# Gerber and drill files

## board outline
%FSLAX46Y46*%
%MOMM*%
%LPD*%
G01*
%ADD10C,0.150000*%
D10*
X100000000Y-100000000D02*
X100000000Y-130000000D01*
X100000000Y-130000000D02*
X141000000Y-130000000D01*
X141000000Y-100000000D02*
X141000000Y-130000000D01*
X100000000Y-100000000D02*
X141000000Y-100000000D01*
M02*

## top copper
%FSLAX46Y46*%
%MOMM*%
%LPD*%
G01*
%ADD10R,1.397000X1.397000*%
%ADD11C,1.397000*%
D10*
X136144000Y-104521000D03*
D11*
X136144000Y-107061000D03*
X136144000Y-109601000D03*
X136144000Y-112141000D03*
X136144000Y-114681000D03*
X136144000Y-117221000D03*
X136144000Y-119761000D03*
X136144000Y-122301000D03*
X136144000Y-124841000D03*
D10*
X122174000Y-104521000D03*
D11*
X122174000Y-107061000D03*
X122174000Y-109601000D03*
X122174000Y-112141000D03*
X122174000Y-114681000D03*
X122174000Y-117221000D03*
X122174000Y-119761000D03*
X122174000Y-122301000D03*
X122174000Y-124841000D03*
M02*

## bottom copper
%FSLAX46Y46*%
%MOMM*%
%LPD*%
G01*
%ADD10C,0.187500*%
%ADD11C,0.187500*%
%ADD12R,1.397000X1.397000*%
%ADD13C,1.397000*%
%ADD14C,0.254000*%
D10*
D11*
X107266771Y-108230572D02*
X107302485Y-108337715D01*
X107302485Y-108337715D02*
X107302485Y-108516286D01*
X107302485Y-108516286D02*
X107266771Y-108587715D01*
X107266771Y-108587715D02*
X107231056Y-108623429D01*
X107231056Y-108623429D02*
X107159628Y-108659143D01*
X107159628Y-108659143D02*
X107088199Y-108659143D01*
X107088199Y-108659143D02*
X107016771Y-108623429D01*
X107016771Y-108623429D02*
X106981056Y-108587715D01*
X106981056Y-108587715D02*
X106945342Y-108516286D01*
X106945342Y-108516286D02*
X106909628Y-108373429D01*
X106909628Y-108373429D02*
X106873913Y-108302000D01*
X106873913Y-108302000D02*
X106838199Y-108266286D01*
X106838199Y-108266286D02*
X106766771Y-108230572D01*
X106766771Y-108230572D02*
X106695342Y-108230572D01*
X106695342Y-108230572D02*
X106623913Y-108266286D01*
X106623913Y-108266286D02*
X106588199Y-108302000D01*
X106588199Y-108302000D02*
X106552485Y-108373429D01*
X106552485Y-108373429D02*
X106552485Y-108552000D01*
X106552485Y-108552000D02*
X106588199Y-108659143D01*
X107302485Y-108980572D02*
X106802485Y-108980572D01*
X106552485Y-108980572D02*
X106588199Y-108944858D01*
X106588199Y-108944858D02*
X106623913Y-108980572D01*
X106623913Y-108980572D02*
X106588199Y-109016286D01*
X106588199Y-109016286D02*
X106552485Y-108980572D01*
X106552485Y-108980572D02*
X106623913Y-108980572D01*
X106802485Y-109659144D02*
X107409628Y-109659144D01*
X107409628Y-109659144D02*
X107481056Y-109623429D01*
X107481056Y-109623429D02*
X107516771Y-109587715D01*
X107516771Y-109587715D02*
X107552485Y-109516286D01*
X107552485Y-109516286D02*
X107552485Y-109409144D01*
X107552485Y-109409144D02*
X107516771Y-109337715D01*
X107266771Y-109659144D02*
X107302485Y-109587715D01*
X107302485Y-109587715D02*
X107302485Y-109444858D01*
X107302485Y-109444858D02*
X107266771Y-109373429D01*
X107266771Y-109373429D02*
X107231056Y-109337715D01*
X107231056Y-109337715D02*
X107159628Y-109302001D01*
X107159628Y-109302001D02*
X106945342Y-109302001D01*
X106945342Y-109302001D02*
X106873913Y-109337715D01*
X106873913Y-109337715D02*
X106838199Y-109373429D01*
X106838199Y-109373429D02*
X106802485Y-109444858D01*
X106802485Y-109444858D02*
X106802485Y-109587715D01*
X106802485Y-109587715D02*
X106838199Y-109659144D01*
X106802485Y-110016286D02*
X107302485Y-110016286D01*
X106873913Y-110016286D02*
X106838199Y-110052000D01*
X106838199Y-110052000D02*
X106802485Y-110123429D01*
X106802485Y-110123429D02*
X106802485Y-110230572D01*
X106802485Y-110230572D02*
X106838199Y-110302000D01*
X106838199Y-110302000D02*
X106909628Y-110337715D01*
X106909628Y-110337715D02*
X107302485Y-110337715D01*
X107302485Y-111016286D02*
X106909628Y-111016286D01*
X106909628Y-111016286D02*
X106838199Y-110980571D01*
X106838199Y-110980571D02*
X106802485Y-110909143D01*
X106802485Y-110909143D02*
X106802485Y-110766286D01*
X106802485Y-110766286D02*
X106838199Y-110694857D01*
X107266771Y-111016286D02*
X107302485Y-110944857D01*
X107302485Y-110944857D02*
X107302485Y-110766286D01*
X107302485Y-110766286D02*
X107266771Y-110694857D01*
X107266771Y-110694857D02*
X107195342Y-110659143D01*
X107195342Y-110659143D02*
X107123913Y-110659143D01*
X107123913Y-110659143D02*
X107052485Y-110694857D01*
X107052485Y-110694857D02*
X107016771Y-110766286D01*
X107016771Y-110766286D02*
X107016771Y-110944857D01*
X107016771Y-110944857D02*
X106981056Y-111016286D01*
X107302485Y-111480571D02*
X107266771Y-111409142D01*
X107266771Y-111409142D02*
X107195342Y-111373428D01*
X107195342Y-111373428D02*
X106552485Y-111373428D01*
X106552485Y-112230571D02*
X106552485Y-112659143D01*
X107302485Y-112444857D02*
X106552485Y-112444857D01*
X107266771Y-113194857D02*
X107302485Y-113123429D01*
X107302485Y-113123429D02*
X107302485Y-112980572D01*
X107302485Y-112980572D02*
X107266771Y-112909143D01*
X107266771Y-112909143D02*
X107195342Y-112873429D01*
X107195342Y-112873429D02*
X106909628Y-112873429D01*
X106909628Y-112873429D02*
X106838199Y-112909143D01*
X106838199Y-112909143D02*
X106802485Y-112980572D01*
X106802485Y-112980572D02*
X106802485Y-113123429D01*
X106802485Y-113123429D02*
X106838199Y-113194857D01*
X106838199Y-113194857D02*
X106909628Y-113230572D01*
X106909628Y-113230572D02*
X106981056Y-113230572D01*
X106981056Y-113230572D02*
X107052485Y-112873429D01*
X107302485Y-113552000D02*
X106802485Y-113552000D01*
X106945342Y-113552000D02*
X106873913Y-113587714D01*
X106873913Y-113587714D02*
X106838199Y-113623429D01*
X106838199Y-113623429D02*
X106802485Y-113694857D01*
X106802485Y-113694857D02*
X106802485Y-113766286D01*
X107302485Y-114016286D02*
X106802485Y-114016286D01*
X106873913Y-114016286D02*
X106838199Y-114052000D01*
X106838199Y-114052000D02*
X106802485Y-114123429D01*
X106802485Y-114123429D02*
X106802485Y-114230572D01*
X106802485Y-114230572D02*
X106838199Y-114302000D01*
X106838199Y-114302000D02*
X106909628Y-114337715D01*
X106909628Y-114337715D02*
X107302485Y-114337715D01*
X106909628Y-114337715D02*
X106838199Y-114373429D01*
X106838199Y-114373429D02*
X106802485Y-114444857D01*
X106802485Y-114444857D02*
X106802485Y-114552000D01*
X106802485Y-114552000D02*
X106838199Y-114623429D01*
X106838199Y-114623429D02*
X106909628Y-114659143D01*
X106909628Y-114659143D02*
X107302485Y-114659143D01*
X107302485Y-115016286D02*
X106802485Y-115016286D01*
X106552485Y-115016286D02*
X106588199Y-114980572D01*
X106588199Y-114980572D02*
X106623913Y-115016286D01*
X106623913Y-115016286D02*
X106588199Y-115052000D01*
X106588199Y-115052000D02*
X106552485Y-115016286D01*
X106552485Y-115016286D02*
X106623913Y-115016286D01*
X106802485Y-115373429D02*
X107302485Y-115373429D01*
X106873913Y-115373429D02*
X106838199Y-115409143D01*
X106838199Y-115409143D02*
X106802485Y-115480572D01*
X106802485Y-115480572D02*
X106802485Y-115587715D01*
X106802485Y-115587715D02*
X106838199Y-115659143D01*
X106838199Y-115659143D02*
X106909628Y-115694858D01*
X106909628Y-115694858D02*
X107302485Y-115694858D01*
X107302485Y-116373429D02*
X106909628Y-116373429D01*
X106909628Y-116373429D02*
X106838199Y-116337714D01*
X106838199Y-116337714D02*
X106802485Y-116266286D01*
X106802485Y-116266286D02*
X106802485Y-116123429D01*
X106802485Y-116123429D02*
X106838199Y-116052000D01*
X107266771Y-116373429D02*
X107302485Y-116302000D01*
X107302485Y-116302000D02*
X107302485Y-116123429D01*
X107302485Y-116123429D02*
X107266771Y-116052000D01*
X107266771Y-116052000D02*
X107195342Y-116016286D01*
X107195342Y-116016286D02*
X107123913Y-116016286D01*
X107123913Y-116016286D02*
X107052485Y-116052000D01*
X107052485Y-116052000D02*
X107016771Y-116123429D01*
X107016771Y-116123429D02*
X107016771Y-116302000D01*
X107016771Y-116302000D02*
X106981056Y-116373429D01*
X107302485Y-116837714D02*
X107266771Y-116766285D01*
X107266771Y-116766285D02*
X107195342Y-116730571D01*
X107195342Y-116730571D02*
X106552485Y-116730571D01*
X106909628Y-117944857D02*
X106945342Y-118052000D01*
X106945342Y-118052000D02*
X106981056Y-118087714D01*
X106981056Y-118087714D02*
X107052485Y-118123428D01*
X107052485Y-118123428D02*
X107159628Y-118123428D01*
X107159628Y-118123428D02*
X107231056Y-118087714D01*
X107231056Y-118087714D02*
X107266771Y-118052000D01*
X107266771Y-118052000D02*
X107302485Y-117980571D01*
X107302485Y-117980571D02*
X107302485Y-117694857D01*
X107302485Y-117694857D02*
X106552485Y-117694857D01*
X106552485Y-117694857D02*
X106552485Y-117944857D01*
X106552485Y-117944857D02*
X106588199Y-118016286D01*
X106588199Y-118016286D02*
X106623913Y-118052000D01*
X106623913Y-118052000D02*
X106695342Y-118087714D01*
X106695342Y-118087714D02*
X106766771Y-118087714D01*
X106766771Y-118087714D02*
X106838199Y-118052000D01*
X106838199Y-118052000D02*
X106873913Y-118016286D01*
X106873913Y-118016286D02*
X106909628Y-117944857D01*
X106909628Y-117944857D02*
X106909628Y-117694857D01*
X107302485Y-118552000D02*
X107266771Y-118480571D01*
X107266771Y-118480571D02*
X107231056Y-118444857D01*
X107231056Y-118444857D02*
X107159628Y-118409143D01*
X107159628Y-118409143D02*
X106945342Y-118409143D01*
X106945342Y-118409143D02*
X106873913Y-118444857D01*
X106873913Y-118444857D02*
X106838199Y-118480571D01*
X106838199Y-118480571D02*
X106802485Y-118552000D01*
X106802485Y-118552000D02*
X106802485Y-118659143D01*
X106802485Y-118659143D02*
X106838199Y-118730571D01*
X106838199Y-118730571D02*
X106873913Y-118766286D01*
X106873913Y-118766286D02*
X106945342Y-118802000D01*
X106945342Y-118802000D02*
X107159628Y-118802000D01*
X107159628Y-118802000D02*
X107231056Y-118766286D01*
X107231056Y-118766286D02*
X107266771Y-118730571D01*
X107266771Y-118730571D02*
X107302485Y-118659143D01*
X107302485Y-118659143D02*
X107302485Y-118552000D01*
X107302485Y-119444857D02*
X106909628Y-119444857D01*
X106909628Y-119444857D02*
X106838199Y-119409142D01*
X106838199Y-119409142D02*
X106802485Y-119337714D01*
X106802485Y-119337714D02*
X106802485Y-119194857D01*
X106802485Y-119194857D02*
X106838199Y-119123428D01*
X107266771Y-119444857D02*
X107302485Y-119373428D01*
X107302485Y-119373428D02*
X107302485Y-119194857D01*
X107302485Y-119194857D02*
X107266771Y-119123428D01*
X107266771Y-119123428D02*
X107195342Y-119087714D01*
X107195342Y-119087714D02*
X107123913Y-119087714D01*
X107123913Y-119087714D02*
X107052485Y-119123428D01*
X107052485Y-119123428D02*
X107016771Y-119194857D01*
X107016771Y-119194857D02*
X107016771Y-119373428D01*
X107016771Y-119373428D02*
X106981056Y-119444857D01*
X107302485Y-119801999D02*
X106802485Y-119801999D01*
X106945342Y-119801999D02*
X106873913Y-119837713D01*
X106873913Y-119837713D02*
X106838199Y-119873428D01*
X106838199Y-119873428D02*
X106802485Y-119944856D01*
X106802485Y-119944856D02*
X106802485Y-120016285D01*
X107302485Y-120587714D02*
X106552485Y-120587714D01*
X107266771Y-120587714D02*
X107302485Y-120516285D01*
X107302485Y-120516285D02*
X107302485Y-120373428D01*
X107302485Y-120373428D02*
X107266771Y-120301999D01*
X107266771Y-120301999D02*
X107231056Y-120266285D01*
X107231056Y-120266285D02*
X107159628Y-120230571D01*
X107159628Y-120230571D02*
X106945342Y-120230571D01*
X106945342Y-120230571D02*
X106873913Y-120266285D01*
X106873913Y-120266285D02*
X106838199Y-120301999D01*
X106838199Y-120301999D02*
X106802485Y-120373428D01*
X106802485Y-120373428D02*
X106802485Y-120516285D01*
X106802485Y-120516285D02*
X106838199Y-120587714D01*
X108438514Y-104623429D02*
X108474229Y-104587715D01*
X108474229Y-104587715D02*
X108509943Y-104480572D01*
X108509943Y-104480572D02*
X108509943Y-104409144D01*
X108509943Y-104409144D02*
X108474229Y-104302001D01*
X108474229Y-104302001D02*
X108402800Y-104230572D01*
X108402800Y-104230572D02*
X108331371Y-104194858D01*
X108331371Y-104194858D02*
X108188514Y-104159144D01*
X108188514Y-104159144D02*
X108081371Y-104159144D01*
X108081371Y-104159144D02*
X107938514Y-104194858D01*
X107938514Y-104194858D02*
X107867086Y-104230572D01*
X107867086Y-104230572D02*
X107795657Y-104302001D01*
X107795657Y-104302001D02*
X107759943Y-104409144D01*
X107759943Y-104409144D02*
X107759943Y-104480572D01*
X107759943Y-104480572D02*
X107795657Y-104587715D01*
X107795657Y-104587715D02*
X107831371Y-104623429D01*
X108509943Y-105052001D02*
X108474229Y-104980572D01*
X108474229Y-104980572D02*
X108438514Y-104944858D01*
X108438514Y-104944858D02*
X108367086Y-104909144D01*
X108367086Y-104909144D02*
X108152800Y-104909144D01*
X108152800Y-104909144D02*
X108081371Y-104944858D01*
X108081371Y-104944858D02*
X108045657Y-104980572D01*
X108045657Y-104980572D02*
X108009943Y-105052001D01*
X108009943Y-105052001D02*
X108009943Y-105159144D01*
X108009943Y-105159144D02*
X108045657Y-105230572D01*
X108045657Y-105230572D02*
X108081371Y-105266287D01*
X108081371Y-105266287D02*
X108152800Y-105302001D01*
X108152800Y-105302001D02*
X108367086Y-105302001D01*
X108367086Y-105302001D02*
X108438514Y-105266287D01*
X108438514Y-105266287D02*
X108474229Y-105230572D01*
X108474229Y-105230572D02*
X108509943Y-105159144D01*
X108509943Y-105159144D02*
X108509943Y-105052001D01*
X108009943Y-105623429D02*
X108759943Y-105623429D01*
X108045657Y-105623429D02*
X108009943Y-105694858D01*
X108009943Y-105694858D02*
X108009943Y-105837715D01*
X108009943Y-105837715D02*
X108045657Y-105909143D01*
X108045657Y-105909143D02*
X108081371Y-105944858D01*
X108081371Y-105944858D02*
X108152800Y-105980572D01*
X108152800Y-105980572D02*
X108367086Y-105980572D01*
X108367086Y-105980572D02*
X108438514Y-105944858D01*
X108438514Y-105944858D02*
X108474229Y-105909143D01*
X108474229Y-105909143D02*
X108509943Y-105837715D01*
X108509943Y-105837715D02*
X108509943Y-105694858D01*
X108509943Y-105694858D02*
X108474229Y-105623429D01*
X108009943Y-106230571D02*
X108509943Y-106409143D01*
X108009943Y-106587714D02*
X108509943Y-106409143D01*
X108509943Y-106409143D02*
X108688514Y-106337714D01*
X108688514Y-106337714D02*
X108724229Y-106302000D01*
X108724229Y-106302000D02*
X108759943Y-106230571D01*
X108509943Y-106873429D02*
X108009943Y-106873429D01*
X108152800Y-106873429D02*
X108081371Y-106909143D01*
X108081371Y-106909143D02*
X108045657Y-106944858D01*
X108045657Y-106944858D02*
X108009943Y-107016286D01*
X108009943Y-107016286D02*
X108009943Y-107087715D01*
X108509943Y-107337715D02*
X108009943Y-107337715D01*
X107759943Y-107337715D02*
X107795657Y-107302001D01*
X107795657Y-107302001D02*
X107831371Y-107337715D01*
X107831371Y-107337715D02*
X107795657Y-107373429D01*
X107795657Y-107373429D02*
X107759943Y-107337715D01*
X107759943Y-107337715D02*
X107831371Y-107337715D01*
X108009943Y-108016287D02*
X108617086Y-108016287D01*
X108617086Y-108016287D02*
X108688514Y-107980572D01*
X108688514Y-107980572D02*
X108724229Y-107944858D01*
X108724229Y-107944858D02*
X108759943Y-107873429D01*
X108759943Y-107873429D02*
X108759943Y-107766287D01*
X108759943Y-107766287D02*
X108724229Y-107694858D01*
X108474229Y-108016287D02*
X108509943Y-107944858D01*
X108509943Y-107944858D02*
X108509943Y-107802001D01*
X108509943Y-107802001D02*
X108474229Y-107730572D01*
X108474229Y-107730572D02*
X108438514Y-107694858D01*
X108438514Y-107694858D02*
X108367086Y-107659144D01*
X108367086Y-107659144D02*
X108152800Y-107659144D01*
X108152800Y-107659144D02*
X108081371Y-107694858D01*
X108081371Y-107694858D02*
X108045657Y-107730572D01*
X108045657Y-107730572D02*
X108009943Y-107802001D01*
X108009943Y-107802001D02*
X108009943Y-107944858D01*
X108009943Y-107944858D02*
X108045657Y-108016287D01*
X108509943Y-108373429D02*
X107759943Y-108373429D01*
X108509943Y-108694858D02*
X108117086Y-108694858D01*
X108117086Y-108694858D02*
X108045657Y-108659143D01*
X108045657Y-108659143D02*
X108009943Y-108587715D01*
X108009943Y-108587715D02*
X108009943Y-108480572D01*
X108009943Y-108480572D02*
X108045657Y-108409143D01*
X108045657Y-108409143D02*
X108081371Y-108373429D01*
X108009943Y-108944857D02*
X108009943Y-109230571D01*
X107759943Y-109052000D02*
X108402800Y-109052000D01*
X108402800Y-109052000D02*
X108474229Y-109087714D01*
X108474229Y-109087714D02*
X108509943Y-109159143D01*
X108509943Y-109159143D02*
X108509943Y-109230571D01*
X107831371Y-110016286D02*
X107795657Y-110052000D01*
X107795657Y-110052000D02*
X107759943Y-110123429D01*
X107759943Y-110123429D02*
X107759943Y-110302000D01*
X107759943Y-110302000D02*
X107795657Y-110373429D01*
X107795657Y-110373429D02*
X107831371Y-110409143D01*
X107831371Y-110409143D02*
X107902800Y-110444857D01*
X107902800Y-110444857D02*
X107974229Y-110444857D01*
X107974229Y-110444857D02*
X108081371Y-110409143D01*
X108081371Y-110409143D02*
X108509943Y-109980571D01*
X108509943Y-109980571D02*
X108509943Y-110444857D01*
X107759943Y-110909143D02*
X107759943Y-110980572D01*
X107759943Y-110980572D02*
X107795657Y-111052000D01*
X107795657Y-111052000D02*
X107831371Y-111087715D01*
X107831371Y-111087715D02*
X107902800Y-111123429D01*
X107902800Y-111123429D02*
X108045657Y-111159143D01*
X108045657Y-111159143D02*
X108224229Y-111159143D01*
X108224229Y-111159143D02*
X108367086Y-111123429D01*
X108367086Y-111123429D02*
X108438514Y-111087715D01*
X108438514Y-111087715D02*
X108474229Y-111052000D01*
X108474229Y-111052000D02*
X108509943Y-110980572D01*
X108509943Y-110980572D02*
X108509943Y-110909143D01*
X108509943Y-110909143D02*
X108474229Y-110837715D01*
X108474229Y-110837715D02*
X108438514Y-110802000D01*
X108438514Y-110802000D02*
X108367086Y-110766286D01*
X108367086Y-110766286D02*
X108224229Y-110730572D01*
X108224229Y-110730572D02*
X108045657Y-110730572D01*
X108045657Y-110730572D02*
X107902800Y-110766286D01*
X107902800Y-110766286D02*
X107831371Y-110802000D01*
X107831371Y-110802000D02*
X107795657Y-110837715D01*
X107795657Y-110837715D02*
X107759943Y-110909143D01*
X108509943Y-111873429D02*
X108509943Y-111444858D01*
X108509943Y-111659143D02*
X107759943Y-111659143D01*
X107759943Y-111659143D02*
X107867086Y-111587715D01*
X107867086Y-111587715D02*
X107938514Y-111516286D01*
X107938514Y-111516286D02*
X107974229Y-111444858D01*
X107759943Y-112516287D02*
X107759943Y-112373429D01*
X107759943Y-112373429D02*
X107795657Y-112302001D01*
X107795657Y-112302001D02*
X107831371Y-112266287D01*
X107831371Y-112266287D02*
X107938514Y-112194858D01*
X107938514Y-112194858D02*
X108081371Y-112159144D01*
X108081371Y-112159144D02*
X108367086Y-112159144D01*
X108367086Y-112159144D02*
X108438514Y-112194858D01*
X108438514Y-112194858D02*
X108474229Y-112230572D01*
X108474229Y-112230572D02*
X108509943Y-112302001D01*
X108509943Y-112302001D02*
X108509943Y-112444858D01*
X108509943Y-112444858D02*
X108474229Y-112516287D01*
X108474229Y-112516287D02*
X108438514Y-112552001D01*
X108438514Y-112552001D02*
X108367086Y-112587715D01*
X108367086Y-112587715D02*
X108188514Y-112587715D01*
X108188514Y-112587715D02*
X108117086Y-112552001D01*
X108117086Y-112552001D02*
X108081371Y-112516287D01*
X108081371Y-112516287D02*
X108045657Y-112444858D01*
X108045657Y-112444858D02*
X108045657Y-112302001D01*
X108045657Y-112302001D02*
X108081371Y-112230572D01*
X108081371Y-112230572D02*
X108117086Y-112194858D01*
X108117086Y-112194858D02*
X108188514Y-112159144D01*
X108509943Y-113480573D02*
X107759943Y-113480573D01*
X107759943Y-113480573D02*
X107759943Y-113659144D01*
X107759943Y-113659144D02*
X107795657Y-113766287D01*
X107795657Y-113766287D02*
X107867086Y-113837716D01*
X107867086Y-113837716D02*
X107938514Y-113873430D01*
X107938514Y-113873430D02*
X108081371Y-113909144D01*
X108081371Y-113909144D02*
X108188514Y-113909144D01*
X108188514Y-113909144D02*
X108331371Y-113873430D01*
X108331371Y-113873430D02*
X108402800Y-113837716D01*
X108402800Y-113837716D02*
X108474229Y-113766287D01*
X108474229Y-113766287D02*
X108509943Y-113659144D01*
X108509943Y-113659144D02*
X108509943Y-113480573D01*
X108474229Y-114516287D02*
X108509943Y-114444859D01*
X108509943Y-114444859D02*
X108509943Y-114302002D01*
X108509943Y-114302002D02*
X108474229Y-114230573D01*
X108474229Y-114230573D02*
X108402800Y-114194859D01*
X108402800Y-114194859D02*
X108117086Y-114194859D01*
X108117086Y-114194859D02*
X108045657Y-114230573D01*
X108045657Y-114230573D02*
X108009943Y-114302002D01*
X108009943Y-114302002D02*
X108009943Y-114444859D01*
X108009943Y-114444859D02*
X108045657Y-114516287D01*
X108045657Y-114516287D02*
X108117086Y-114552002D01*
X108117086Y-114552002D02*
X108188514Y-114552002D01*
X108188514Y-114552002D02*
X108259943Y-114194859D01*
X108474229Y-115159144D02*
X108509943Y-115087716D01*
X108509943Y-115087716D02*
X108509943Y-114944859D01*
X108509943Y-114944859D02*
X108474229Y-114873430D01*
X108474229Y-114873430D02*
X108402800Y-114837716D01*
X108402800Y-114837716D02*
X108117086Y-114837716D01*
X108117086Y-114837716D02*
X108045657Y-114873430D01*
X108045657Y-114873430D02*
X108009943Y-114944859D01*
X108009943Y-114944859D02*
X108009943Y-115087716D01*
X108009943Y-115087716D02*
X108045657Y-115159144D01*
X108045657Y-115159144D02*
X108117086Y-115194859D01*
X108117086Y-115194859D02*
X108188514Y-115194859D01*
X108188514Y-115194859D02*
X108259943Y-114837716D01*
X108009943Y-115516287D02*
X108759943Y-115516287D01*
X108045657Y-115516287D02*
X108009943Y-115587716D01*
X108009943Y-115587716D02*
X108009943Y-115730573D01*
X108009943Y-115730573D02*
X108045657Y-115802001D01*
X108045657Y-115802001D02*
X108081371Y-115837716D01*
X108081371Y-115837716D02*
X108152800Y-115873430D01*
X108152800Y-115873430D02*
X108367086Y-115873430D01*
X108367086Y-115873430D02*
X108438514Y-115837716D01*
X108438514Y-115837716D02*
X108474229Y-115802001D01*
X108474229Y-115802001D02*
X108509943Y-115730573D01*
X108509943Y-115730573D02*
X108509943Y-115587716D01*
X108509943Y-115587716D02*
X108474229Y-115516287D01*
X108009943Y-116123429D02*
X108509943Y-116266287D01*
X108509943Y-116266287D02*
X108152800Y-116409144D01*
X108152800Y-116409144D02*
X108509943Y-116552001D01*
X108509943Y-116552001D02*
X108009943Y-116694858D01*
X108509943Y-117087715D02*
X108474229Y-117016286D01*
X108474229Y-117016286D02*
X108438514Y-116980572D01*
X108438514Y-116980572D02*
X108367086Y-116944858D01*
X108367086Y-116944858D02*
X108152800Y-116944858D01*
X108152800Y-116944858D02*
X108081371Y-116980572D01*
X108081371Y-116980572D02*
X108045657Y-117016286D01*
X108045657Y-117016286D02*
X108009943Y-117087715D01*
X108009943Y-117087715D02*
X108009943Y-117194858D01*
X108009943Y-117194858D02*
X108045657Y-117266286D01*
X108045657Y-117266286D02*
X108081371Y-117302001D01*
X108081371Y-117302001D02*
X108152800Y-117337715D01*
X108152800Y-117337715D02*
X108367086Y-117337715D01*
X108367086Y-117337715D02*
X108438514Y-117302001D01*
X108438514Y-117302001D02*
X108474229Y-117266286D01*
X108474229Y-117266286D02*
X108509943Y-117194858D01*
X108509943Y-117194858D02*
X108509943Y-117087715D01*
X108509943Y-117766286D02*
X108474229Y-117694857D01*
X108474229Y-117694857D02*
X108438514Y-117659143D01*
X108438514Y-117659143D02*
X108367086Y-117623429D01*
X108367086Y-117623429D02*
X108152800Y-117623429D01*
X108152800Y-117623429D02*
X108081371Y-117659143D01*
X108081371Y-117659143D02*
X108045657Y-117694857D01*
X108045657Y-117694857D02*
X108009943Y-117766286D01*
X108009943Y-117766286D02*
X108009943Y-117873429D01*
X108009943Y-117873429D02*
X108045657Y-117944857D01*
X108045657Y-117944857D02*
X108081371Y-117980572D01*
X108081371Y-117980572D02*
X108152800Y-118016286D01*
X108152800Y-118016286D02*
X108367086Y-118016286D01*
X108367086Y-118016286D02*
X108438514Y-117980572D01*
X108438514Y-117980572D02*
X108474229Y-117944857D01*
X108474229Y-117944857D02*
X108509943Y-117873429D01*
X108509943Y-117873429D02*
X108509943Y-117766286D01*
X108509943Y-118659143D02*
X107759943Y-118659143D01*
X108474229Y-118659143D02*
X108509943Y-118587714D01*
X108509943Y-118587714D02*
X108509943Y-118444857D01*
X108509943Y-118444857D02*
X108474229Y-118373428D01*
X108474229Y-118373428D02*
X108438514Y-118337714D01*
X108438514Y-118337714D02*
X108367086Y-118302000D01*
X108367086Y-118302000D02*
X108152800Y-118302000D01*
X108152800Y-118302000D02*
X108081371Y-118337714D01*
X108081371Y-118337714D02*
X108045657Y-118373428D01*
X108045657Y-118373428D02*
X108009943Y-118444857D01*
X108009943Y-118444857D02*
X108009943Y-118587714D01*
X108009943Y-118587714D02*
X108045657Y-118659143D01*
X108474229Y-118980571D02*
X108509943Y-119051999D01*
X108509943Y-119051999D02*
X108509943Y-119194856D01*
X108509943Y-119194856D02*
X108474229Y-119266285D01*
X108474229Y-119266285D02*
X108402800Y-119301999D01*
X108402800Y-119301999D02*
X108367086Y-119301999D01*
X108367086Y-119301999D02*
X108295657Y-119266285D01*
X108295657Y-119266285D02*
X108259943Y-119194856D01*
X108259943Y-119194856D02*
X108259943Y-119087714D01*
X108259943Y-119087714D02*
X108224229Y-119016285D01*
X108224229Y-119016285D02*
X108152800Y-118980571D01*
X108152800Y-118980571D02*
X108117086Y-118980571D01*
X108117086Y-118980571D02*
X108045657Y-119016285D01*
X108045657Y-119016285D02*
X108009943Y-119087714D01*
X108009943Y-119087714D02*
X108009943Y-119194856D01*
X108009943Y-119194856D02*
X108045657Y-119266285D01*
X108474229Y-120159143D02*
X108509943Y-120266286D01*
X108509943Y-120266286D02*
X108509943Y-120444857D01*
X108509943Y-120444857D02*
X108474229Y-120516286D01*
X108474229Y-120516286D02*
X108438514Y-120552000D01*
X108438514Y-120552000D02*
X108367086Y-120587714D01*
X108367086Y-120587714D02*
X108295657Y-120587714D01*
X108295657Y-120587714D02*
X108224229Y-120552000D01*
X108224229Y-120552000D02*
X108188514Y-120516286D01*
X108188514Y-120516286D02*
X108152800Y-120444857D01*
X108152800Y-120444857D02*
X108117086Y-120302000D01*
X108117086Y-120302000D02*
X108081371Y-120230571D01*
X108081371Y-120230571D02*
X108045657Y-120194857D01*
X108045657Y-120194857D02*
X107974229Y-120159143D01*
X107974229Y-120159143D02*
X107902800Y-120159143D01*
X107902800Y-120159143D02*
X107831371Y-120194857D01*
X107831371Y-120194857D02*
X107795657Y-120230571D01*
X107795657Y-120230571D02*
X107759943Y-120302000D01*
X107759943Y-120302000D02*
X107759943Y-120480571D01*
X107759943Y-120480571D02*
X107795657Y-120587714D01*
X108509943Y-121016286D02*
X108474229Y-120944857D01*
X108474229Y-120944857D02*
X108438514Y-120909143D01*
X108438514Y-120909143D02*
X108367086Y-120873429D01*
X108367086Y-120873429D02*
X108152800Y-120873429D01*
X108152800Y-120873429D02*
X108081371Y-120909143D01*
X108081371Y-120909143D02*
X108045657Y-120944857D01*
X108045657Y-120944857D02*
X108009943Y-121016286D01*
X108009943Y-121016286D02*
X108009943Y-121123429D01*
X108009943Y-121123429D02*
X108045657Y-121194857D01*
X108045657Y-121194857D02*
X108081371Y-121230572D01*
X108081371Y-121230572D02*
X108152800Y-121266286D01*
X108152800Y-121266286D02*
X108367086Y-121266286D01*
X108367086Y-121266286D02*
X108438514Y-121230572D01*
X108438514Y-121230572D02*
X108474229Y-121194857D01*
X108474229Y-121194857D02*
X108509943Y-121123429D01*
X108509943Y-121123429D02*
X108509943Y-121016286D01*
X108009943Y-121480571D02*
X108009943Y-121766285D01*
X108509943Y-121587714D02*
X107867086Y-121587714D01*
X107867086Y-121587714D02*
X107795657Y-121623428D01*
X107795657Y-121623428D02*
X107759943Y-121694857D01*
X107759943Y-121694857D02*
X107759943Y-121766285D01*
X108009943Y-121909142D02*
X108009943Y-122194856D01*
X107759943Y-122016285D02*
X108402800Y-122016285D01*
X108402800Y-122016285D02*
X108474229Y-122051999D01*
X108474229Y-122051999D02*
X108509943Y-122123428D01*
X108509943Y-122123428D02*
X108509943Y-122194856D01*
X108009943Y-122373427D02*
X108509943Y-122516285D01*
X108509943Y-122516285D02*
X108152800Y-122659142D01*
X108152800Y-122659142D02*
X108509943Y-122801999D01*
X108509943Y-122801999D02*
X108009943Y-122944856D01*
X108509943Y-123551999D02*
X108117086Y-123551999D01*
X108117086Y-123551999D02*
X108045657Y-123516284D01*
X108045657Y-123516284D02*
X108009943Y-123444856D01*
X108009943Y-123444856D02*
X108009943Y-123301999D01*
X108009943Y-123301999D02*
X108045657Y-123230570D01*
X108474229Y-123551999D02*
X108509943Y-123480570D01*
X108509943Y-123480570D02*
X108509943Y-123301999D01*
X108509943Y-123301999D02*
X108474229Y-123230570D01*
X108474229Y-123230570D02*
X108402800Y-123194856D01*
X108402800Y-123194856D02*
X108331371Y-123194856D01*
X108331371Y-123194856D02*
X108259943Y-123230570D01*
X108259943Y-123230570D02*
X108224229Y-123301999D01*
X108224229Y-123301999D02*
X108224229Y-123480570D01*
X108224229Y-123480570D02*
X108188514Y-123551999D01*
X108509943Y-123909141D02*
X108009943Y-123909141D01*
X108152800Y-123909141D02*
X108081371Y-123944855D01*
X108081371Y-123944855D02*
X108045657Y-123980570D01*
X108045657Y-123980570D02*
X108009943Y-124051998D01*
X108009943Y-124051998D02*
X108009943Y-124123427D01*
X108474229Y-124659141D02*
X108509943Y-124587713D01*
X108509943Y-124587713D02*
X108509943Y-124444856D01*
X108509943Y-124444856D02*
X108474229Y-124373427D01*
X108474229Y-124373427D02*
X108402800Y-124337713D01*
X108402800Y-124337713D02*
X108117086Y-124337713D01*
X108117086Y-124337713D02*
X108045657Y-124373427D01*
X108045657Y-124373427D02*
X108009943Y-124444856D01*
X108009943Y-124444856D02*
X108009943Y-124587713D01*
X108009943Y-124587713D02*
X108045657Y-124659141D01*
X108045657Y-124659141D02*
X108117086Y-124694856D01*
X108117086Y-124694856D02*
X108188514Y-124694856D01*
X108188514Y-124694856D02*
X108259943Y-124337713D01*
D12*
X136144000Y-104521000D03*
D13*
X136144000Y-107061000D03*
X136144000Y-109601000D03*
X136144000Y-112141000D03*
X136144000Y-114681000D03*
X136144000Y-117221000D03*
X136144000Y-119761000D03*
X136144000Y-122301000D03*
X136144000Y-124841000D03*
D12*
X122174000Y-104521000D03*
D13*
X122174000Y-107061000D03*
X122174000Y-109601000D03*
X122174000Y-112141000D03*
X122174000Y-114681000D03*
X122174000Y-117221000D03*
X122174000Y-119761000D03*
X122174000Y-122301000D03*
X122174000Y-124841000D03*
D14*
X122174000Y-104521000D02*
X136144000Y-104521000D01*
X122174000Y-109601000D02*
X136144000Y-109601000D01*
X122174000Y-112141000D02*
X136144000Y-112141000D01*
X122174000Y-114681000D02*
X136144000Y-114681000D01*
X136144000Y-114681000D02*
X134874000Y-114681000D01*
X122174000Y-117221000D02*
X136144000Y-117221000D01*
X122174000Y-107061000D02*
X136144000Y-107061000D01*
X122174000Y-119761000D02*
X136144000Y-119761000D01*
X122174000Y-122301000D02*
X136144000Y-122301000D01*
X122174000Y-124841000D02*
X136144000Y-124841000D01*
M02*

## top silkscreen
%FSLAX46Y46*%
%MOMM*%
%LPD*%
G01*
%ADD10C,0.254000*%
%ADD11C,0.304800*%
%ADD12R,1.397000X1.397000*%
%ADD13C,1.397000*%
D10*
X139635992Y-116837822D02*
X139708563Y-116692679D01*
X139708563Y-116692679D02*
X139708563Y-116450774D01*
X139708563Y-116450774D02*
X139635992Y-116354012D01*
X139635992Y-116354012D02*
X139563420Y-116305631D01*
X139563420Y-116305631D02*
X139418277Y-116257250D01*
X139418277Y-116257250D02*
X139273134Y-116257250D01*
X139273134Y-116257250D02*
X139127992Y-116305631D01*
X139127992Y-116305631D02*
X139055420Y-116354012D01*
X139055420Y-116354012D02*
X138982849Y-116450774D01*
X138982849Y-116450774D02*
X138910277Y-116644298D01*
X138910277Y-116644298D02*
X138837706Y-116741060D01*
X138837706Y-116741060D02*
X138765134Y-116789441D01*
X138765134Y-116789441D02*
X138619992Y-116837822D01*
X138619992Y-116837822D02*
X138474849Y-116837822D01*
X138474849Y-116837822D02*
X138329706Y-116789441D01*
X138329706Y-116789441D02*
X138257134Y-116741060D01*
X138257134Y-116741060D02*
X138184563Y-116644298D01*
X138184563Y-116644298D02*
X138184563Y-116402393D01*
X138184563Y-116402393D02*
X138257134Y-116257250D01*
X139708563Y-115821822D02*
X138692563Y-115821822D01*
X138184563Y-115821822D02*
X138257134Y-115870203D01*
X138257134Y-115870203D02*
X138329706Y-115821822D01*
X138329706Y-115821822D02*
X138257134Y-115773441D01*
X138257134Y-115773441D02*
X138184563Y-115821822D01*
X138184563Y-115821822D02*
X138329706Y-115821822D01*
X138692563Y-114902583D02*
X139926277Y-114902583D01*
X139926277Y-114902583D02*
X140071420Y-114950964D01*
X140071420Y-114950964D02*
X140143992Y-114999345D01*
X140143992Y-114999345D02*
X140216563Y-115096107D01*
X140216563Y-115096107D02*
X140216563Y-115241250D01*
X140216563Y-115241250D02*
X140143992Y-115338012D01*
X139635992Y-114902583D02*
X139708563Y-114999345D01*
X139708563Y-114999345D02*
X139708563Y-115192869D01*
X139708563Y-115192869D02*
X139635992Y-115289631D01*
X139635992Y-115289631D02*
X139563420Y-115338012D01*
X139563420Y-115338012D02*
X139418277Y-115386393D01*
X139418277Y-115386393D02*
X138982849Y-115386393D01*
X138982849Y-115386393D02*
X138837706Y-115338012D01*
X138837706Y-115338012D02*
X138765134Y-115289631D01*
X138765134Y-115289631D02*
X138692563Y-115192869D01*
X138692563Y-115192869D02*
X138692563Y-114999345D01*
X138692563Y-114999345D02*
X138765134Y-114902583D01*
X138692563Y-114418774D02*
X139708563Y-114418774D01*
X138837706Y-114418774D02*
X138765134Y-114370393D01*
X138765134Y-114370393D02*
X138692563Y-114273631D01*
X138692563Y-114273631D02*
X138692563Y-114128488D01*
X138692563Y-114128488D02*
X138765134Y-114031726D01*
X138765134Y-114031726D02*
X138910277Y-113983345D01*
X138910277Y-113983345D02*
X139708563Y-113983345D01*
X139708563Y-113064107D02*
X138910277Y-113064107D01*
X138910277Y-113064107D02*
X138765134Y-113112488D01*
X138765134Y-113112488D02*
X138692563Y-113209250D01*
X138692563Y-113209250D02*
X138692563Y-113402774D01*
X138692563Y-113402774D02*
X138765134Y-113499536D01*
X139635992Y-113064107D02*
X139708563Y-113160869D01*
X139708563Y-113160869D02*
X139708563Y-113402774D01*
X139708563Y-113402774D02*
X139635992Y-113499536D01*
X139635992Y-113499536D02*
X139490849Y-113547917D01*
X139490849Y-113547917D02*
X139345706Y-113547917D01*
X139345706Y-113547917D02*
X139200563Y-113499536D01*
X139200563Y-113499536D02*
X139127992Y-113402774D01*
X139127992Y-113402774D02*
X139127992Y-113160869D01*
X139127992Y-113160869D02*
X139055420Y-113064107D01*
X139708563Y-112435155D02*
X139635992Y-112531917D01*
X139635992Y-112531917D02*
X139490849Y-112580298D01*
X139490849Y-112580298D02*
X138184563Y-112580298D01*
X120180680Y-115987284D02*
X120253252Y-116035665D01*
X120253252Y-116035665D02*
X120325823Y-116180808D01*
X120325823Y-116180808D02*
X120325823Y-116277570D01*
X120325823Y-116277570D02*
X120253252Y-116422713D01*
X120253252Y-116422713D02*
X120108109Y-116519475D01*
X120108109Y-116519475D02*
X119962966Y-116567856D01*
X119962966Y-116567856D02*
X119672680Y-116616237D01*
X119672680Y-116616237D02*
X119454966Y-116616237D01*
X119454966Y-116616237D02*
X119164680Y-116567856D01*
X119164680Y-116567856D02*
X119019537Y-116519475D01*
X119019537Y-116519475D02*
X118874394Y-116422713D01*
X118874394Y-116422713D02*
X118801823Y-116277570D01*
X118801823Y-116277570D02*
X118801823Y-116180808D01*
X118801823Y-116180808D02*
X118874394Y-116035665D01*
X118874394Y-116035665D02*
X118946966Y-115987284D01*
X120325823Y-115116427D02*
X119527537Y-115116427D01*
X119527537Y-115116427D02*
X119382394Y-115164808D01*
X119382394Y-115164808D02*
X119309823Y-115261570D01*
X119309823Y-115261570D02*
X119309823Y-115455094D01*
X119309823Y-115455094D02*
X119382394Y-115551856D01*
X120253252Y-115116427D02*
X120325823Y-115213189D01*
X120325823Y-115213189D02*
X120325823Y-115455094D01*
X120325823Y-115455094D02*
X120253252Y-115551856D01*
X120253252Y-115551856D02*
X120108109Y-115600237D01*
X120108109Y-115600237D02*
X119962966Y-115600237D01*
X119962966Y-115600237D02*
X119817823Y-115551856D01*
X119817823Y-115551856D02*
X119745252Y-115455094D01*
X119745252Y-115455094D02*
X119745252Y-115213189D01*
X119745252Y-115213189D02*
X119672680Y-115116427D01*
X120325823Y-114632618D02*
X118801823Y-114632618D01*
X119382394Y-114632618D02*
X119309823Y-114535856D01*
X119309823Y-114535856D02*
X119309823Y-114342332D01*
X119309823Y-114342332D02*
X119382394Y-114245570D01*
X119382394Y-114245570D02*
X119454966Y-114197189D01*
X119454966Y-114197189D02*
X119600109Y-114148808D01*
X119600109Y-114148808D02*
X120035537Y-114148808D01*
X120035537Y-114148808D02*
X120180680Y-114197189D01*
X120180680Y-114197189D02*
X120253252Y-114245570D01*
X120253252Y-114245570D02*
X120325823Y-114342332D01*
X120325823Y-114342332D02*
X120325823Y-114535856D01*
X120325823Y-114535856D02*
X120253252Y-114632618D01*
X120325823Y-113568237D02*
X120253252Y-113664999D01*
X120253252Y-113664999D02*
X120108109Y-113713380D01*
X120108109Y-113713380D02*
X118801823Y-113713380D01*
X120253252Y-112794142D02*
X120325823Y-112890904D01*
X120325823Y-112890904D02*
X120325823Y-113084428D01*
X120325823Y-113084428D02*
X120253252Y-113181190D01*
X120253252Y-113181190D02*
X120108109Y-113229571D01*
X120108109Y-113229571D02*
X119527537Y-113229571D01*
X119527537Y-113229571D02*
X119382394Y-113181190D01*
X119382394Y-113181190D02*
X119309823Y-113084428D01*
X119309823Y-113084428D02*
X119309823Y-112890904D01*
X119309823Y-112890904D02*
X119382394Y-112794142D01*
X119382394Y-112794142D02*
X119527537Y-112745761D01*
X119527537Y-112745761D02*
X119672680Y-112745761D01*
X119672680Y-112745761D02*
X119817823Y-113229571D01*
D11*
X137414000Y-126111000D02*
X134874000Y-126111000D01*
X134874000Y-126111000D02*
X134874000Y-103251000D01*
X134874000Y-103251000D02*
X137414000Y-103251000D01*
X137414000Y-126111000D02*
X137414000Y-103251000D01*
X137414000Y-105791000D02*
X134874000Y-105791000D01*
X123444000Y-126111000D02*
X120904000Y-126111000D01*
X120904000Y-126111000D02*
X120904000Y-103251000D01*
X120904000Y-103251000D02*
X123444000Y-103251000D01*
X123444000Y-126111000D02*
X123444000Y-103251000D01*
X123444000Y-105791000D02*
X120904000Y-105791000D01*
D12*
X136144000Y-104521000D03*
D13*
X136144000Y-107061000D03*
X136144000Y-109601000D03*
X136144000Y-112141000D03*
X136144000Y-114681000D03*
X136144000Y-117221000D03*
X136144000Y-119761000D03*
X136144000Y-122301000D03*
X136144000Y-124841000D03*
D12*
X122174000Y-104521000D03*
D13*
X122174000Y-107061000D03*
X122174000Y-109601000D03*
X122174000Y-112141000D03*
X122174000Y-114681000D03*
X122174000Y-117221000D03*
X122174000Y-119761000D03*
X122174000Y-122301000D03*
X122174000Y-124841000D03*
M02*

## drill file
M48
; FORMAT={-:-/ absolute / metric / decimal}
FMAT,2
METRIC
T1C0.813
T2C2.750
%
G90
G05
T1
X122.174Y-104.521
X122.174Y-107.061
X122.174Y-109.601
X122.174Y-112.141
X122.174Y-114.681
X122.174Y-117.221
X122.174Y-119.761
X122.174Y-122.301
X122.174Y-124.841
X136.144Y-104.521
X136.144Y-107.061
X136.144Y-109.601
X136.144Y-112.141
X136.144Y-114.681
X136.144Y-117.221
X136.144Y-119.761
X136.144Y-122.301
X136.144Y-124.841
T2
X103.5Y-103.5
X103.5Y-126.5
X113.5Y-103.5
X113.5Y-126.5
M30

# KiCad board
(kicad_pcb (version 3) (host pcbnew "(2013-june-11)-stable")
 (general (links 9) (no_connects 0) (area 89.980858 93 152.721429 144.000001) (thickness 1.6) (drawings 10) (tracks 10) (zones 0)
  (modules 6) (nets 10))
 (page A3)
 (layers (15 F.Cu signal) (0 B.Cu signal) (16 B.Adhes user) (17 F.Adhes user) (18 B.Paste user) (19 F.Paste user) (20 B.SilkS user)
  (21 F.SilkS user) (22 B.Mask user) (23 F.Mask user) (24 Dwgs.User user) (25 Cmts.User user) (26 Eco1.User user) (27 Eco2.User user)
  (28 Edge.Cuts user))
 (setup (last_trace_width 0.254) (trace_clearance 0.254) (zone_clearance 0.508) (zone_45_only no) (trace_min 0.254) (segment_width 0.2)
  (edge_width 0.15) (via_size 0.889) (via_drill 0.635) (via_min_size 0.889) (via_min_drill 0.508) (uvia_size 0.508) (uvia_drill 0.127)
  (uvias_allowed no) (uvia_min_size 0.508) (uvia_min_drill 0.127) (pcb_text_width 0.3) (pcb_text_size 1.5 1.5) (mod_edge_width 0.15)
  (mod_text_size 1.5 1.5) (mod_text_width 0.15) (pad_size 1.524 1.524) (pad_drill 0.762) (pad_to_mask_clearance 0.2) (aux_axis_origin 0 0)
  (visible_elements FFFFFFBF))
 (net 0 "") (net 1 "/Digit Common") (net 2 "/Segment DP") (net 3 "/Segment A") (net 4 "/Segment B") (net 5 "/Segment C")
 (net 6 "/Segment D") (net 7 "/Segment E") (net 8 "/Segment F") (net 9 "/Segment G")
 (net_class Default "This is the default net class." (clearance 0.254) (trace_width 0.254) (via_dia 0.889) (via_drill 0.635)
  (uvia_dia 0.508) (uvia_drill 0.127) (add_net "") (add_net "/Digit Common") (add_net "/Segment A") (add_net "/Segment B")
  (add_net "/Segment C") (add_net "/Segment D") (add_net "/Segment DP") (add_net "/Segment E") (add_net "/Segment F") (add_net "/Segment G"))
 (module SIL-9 (layer F.Cu) (at 136.144 114.681 270)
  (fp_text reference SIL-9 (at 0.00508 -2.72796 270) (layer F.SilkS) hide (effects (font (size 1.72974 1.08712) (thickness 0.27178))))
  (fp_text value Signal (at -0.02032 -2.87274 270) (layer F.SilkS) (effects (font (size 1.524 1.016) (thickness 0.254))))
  (fp_line (start 11.43 -1.27) (end 11.43 1.27) (layer F.SilkS) (width 0.3048))
  (fp_line (start 11.43 1.27) (end -11.43 1.27) (layer F.SilkS) (width 0.3048))
  (fp_line (start -11.43 1.27) (end -11.43 -1.27) (layer F.SilkS) (width 0.3048))
  (fp_line (start 11.43 -1.27) (end -11.43 -1.27) (layer F.SilkS) (width 0.3048))
  (fp_line (start -8.89 -1.27) (end -8.89 1.27) (layer F.SilkS) (width 0.3048))
  (pad 1 thru_hole rect (at -10.16 0 270) (size 1.397 1.397) (drill 0.8128) (layers *.Cu *.Mask F.SilkS) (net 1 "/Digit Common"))
  (pad 2 thru_hole circle (at -7.62 0 270) (size 1.397 1.397) (drill 0.8128) (layers *.Cu *.Mask F.SilkS) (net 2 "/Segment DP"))
  (pad 3 thru_hole circle (at -5.08 0 270) (size 1.397 1.397) (drill 0.8128) (layers *.Cu *.Mask F.SilkS) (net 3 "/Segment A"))
  (pad 4 thru_hole circle (at -2.54 0 270) (size 1.397 1.397) (drill 0.8128) (layers *.Cu *.Mask F.SilkS) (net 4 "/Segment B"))
  (pad 5 thru_hole circle (at 0 0 270) (size 1.397 1.397) (drill 0.8128) (layers *.Cu *.Mask F.SilkS) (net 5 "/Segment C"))
  (pad 6 thru_hole circle (at 2.54 0 270) (size 1.397 1.397) (drill 0.8128) (layers *.Cu *.Mask F.SilkS) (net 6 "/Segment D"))
  (pad 7 thru_hole circle (at 5.08 0 270) (size 1.397 1.397) (drill 0.8128) (layers *.Cu *.Mask F.SilkS) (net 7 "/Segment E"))
  (pad 8 thru_hole circle (at 7.62 0 270) (size 1.397 1.397) (drill 0.8128) (layers *.Cu *.Mask F.SilkS) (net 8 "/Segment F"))
  (pad 9 thru_hole circle (at 10.16 0 270) (size 1.397 1.397) (drill 0.8128) (layers *.Cu *.Mask F.SilkS) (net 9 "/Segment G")))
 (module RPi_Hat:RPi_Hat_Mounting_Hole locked (layer B.Cu) (at 113.5 126.5)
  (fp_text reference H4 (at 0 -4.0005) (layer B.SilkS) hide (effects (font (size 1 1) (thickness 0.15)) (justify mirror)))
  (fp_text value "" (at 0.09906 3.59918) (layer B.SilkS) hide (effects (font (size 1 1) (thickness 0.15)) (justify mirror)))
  (pad "" np_thru_hole circle (at 0 0) (size 2.75 2.75) (drill 2.75) (layers *.Cu *.Mask) (solder_mask_margin 1.725) (clearance 1.725)))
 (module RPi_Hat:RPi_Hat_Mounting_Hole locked (layer B.Cu) (at 103.5 103.5)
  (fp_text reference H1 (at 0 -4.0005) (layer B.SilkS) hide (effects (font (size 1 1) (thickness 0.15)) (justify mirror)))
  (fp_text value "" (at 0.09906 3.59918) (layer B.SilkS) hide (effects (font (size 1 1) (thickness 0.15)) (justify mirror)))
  (pad "" np_thru_hole circle (at 0 0) (size 2.75 2.75) (drill 2.75) (layers *.Cu *.Mask) (solder_mask_margin 1.725) (clearance 1.725)))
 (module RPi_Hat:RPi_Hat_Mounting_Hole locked (layer B.Cu) (at 113.5 103.5)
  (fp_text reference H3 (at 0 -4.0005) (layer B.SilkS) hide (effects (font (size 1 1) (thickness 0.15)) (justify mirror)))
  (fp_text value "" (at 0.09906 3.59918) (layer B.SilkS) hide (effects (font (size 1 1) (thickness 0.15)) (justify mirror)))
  (pad "" np_thru_hole circle (at 0 0) (size 2.75 2.75) (drill 2.75) (layers *.Cu *.Mask) (solder_mask_margin 1.725) (clearance 1.725)))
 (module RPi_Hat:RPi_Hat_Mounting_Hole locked (layer B.Cu) (at 103.5 126.5)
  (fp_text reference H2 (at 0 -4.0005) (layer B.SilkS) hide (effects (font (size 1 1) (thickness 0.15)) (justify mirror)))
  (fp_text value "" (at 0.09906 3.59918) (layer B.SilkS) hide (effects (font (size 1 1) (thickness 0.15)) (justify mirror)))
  (pad "" np_thru_hole circle (at 0 0) (size 2.75 2.75) (drill 2.75) (layers *.Cu *.Mask) (solder_mask_margin 1.725) (clearance 1.725)))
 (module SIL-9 (layer F.Cu) (at 122.174 114.681 270)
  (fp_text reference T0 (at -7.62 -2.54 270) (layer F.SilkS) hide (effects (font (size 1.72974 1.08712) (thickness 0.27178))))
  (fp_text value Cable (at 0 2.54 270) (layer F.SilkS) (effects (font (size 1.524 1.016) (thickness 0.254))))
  (fp_line (start 11.43 -1.27) (end 11.43 1.27) (layer F.SilkS) (width 0.3048))
  (fp_line (start 11.43 1.27) (end -11.43 1.27) (layer F.SilkS) (width 0.3048))
  (fp_line (start -11.43 1.27) (end -11.43 -1.27) (layer F.SilkS) (width 0.3048))
  (fp_line (start 11.43 -1.27) (end -11.43 -1.27) (layer F.SilkS) (width 0.3048))
  (fp_line (start -8.89 -1.27) (end -8.89 1.27) (layer F.SilkS) (width 0.3048))
  (pad 1 thru_hole rect (at -10.16 0 270) (size 1.397 1.397) (drill 0.8128) (layers *.Cu *.Mask F.SilkS) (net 1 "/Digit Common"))
  (pad 2 thru_hole circle (at -7.62 0 270) (size 1.397 1.397) (drill 0.8128) (layers *.Cu *.Mask F.SilkS) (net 2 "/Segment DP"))
  (pad 3 thru_hole circle (at -5.08 0 270) (size 1.397 1.397) (drill 0.8128) (layers *.Cu *.Mask F.SilkS) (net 3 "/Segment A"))
  (pad 4 thru_hole circle (at -2.54 0 270) (size 1.397 1.397) (drill 0.8128) (layers *.Cu *.Mask F.SilkS) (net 4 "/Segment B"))
  (pad 5 thru_hole circle (at 0 0 270) (size 1.397 1.397) (drill 0.8128) (layers *.Cu *.Mask F.SilkS) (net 5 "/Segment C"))
  (pad 6 thru_hole circle (at 2.54 0 270) (size 1.397 1.397) (drill 0.8128) (layers *.Cu *.Mask F.SilkS) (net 6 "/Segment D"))
  (pad 7 thru_hole circle (at 5.08 0 270) (size 1.397 1.397) (drill 0.8128) (layers *.Cu *.Mask F.SilkS) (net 7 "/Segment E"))
  (pad 8 thru_hole circle (at 7.62 0 270) (size 1.397 1.397) (drill 0.8128) (layers *.Cu *.Mask F.SilkS) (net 8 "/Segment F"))
  (pad 9 thru_hole circle (at 10.16 0 270) (size 1.397 1.397) (drill 0.8128) (layers *.Cu *.Mask F.SilkS) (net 9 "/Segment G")))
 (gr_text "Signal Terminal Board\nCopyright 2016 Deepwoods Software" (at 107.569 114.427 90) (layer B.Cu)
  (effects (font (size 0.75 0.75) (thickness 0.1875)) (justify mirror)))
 (gr_line (start 100 100) (end 100 130) (angle 90) (layer Edge.Cuts) (width 0.15))
 (gr_line (start 100 130) (end 141 130) (angle 90) (layer Edge.Cuts) (width 0.15))
 (gr_line (start 141 100) (end 141 130) (angle 90) (layer Edge.Cuts) (width 0.15))
 (gr_line (start 100 100) (end 141 100) (angle 90) (layer Edge.Cuts) (width 0.15))
 (segment (start 122.174 104.521) (end 136.144 104.521) (width 0.254) (layer B.Cu) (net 1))
 (segment (start 122.174 109.601) (end 136.144 109.601) (width 0.254) (layer B.Cu) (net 3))
 (segment (start 122.174 112.141) (end 136.144 112.141) (width 0.254) (layer B.Cu) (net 4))
 (segment (start 122.174 114.681) (end 136.144 114.681) (width 0.254) (layer B.Cu) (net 5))
 (segment (start 136.144 114.681) (end 134.874 114.681) (width 0.254) (layer B.Cu) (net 5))
 (segment (start 122.174 117.221) (end 136.144 117.221) (width 0.254) (layer B.Cu) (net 6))
 (segment (start 122.174 107.061) (end 136.144 107.061) (width 0.254) (layer B.Cu) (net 2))
 (segment (start 122.174 119.761) (end 136.144 119.761) (width 0.254) (layer B.Cu) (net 7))
 (segment (start 122.174 122.301) (end 136.144 122.301) (width 0.254) (layer B.Cu) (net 8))
 (segment (start 122.174 124.841) (end 136.144 124.841) (width 0.254) (layer B.Cu) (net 9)))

